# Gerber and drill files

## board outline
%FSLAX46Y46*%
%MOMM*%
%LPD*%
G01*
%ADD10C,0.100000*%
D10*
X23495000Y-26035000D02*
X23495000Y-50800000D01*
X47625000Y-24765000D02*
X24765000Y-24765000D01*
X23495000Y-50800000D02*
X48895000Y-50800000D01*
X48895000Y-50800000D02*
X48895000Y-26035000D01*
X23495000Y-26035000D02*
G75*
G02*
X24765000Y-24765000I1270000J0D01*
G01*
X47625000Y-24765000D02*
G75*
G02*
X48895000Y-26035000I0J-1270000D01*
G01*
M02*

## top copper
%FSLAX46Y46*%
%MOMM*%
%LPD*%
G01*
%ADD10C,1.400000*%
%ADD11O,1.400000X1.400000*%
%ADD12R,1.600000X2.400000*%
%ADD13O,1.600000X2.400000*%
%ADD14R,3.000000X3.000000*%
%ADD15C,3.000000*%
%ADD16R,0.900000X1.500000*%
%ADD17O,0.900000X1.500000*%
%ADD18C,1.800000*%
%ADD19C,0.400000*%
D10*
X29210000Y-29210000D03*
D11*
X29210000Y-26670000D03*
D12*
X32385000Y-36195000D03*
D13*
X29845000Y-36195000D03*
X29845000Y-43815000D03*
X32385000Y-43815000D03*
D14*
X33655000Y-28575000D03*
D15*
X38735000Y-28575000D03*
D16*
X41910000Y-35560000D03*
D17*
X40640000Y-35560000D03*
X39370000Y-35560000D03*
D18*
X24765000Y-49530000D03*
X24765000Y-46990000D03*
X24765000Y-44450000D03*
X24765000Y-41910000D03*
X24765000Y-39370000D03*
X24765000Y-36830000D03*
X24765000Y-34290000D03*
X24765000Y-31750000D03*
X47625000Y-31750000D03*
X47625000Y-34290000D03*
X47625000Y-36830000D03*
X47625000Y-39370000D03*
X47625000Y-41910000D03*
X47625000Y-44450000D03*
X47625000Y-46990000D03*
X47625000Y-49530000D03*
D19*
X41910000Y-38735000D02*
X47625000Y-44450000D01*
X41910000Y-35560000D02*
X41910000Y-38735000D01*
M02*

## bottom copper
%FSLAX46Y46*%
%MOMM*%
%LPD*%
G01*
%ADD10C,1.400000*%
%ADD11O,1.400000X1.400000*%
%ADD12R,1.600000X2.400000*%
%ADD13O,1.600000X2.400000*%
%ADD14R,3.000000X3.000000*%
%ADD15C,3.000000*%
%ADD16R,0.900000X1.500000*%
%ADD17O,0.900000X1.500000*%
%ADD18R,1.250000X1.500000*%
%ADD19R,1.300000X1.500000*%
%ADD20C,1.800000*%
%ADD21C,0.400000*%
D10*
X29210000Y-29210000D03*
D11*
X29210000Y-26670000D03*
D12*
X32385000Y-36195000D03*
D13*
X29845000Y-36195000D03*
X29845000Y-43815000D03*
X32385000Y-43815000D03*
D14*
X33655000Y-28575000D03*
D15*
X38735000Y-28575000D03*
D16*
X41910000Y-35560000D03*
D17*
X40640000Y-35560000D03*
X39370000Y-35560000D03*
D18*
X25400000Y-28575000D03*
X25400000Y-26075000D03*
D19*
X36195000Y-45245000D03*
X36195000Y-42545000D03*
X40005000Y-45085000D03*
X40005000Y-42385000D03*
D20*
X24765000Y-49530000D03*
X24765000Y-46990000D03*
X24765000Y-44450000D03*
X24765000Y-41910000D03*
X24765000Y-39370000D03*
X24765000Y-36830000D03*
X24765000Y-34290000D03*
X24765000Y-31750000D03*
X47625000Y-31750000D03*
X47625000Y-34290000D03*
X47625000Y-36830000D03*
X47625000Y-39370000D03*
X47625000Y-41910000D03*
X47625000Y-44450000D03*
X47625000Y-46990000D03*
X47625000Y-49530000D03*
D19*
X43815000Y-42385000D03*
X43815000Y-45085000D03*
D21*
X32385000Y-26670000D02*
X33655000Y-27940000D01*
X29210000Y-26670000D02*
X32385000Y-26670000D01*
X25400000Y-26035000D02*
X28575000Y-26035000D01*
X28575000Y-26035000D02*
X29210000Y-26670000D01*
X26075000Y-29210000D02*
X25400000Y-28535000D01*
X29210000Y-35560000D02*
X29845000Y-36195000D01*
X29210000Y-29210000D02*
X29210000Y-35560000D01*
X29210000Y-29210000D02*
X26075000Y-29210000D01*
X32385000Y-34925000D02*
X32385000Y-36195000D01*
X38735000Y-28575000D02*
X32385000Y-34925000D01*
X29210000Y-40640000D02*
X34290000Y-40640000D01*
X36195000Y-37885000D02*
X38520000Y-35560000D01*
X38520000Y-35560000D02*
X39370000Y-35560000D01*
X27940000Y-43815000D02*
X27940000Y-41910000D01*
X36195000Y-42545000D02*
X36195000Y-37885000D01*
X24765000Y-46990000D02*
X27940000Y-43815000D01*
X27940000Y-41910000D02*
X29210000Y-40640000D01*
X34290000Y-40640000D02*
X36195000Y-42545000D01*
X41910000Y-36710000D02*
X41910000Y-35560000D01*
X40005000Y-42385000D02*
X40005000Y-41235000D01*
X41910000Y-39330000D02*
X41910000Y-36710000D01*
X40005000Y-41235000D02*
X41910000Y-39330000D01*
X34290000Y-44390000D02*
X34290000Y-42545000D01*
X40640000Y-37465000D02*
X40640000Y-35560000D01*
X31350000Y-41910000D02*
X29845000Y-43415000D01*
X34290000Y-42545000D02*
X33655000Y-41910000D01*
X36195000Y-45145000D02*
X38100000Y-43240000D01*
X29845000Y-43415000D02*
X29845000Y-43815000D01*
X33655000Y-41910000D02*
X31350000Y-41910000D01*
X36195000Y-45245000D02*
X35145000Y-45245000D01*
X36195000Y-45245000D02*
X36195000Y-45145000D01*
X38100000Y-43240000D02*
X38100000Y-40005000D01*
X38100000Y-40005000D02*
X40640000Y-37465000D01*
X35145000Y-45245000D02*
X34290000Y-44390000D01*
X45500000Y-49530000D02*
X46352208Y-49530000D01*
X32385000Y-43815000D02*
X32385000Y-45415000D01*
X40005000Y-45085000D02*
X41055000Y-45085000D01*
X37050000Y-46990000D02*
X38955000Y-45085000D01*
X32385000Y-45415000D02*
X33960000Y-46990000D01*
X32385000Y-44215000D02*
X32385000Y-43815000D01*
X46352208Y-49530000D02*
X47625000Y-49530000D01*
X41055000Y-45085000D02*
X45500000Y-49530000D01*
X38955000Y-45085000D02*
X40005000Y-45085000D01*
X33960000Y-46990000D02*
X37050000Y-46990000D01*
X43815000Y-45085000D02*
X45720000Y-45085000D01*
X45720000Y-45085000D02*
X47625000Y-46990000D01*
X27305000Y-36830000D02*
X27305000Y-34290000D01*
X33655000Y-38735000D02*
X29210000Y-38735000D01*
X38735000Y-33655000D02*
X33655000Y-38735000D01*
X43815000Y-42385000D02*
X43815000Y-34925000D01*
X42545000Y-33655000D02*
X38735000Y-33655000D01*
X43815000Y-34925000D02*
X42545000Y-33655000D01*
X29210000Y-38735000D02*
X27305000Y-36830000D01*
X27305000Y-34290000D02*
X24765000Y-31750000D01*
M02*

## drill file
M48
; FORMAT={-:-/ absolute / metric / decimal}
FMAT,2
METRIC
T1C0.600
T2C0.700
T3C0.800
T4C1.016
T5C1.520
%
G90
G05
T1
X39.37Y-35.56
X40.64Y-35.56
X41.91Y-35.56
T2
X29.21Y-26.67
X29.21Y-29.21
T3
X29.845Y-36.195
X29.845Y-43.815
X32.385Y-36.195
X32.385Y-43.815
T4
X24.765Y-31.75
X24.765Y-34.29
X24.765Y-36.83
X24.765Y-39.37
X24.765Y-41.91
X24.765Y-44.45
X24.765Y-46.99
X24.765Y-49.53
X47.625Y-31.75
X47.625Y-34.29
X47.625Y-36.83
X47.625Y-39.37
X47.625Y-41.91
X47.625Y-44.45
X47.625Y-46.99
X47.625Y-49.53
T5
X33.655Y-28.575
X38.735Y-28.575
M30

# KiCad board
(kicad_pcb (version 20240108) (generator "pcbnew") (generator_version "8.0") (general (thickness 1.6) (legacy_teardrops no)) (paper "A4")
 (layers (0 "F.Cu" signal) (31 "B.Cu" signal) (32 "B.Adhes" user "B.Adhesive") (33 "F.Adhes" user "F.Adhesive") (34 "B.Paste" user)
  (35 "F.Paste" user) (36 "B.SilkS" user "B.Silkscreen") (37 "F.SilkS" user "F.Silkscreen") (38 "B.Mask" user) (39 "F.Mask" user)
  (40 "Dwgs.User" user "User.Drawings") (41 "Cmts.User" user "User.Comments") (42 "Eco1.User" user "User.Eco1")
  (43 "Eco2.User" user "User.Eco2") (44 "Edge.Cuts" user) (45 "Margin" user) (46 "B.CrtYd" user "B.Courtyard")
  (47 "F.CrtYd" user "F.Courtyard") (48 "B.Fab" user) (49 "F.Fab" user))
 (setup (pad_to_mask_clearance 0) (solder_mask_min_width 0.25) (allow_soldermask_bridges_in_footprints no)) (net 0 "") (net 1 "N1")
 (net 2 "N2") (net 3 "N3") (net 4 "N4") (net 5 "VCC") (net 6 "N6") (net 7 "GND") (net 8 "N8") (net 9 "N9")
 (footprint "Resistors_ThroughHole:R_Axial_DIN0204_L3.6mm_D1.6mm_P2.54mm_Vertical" (layer "F.Cu") (at 29.21 29.21 90)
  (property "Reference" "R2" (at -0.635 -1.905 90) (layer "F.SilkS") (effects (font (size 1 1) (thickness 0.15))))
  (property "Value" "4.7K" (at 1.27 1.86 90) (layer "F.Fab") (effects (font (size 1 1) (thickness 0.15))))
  (pad "1" thru_hole circle (at 0 0 90) (size 1.4 1.4) (drill 0.7) (layers "*.Cu" "*.Mask") (remove_unused_layers no) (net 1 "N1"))
  (pad "2" thru_hole oval (at 2.54 0 90) (size 1.4 1.4) (drill 0.7) (layers "*.Cu" "*.Mask") (remove_unused_layers no) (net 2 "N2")))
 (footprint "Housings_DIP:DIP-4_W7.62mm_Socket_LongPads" (layer "F.Cu") (at 32.385 36.195 -90)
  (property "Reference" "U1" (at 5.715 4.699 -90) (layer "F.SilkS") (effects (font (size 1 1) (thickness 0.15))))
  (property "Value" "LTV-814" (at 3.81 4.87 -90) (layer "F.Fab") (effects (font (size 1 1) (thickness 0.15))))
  (pad "1" thru_hole rect (at 0 0 270) (size 2.4 1.6) (drill 0.8) (layers "*.Cu" "*.Mask") (remove_unused_layers no) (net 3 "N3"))
  (pad "2" thru_hole oval (at 0 2.54 270) (size 2.4 1.6) (drill 0.8) (layers "*.Cu" "*.Mask") (remove_unused_layers no) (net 1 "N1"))
  (pad "3" thru_hole oval (at 7.62 2.54 270) (size 2.4 1.6) (drill 0.8) (layers "*.Cu" "*.Mask") (remove_unused_layers no) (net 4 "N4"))
  (pad "4" thru_hole oval (at 7.62 0 270) (size 2.4 1.6) (drill 0.8) (layers "*.Cu" "*.Mask") (remove_unused_layers no) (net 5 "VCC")))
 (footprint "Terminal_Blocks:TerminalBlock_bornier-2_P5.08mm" (layer "F.Cu") (at 33.655 28.575)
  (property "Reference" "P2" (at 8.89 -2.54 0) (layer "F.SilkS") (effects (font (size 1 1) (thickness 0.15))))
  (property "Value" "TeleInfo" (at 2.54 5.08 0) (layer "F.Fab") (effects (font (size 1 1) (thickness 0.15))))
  (pad "1" thru_hole rect (at 0 0) (size 3 3) (drill 1.52) (layers "*.Cu" "*.Mask") (remove_unused_layers no) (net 2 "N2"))
  (pad "2" thru_hole circle (at 5.08 0) (size 3 3) (drill 1.52) (layers "*.Cu" "*.Mask") (remove_unused_layers no) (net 3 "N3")))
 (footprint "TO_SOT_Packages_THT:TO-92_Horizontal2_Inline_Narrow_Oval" (layer "F.Cu") (at 41.91 35.56 180)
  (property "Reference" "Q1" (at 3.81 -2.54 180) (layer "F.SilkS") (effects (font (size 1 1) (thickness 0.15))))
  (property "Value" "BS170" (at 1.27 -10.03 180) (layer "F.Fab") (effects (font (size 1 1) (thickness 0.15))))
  (pad "1" thru_hole rect (at 0 0) (size 0.9 1.5) (drill 0.6) (layers "*.Cu" "*.Mask") (remove_unused_layers no) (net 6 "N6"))
  (pad "2" thru_hole oval (at 1.27 0) (size 0.9 1.5) (drill 0.6) (layers "*.Cu" "*.Mask") (remove_unused_layers no) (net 4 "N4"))
  (pad "3" thru_hole oval (at 2.54 0) (size 0.9 1.5) (drill 0.6) (layers "*.Cu" "*.Mask") (remove_unused_layers no) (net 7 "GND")))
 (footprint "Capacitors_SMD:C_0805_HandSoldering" (layer "B.Cu") (at 25.4 27.325 90)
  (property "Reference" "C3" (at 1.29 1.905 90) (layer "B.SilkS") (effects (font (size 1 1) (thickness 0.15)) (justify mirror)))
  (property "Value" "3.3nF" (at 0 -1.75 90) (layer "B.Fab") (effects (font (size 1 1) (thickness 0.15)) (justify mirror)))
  (pad "1" smd rect (at -1.25 0 90) (size 1.5 1.25) (layers "B.Cu" "B.Paste" "B.Mask") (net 1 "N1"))
  (pad "2" smd rect (at 1.25 0 90) (size 1.5 1.25) (layers "B.Cu" "B.Paste" "B.Mask") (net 2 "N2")))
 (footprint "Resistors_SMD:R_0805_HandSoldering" (layer "B.Cu") (at 36.195 43.895 90)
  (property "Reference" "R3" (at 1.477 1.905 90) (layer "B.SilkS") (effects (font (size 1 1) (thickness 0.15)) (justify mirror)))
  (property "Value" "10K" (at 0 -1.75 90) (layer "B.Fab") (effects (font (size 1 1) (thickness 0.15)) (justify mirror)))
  (pad "1" smd rect (at -1.35 0 90) (size 1.5 1.3) (layers "B.Cu" "B.Paste" "B.Mask") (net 4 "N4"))
  (pad "2" smd rect (at 1.35 0 90) (size 1.5 1.3) (layers "B.Cu" "B.Paste" "B.Mask") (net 7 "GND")))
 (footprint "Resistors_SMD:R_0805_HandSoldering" (layer "B.Cu") (at 40.005 43.735 90)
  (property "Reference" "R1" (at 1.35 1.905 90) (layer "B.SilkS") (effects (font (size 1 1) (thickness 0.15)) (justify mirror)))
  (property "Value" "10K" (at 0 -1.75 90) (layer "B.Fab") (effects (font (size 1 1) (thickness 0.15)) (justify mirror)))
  (pad "1" smd rect (at -1.35 0 90) (size 1.5 1.3) (layers "B.Cu" "B.Paste" "B.Mask") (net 5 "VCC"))
  (pad "2" smd rect (at 1.35 0 90) (size 1.5 1.3) (layers "B.Cu" "B.Paste" "B.Mask") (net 6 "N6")))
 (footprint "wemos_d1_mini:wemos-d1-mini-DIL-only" (layer "B.Cu") (at 36.195 40.64 90)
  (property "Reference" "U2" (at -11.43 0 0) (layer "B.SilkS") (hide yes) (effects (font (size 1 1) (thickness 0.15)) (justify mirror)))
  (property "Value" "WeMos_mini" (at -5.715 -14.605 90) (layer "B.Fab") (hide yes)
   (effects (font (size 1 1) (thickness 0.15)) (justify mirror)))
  (pad "1" thru_hole circle (at -8.89 -11.43 90) (size 1.8 1.8) (drill 1.016) (layers "*.Cu" "*.Mask") (remove_unused_layers no))
  (pad "2" thru_hole circle (at -6.35 -11.43 90) (size 1.8 1.8) (drill 1.016) (layers "*.Cu" "*.Mask") (remove_unused_layers no)
   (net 7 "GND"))
  (pad "3" thru_hole circle (at -3.81 -11.43 90) (size 1.8 1.8) (drill 1.016) (layers "*.Cu" "*.Mask") (remove_unused_layers no))
  (pad "4" thru_hole circle (at -1.27 -11.43 90) (size 1.8 1.8) (drill 1.016) (layers "*.Cu" "*.Mask") (remove_unused_layers no))
  (pad "5" thru_hole circle (at 1.27 -11.43 90) (size 1.8 1.8) (drill 1.016) (layers "*.Cu" "*.Mask") (remove_unused_layers no))
  (pad "6" thru_hole circle (at 3.81 -11.43 90) (size 1.8 1.8) (drill 1.016) (layers "*.Cu" "*.Mask") (remove_unused_layers no))
  (pad "7" thru_hole circle (at 6.35 -11.43 90) (size 1.8 1.8) (drill 1.016) (layers "*.Cu" "*.Mask") (remove_unused_layers no))
  (pad "8" thru_hole circle (at 8.89 -11.43 90) (size 1.8 1.8) (drill 1.016) (layers "*.Cu" "*.Mask") (remove_unused_layers no) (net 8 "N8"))
  (pad "9" thru_hole circle (at 8.89 11.43 90) (size 1.8 1.8) (drill 1.016) (layers "*.Cu" "*.Mask") (remove_unused_layers no))
  (pad "10" thru_hole circle (at 6.35 11.43 90) (size 1.8 1.8) (drill 1.016) (layers "*.Cu" "*.Mask") (remove_unused_layers no))
  (pad "11" thru_hole circle (at 3.81 11.43 90) (size 1.8 1.8) (drill 1.016) (layers "*.Cu" "*.Mask") (remove_unused_layers no))
  (pad "12" thru_hole circle (at 1.27 11.43 90) (size 1.8 1.8) (drill 1.016) (layers "*.Cu" "*.Mask") (remove_unused_layers no))
  (pad "13" thru_hole circle (at -1.27 11.43 90) (size 1.8 1.8) (drill 1.016) (layers "*.Cu" "*.Mask") (remove_unused_layers no))
  (pad "14" thru_hole circle (at -3.81 11.43 90) (size 1.8 1.8) (drill 1.016) (layers "*.Cu" "*.Mask") (remove_unused_layers no)
   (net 6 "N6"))
  (pad "15" thru_hole circle (at -6.35 11.43 90) (size 1.8 1.8) (drill 1.016) (layers "*.Cu" "*.Mask") (remove_unused_layers no)
   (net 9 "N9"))
  (pad "16" thru_hole circle (at -8.89 11.43 90) (size 1.8 1.8) (drill 1.016) (layers "*.Cu" "*.Mask") (remove_unused_layers no)
   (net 5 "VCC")))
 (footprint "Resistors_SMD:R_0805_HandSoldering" (layer "B.Cu") (at 43.815 43.735 -90)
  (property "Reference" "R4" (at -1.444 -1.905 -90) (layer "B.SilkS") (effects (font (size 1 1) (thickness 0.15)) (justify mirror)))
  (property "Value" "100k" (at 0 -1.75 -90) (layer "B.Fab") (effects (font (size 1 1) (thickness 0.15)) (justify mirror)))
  (pad "1" smd rect (at -1.35 0 270) (size 1.5 1.3) (layers "B.Cu" "B.Paste" "B.Mask") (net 8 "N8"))
  (pad "2" smd rect (at 1.35 0 270) (size 1.5 1.3) (layers "B.Cu" "B.Paste" "B.Mask") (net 9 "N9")))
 (gr_line (start 23.495 26.035) (end 23.495 50.8) (stroke (width 0.1) (type solid)) (layer "Edge.Cuts"))
 (gr_line (start 47.625 24.765) (end 24.765 24.765) (stroke (width 0.1) (type solid)) (layer "Edge.Cuts"))
 (gr_line (start 23.495 50.8) (end 48.895 50.8) (stroke (width 0.1) (type solid)) (layer "Edge.Cuts"))
 (gr_line (start 48.895 50.8) (end 48.895 26.035) (stroke (width 0.1) (type solid)) (layer "Edge.Cuts"))
 (gr_arc (start 23.495 26.035) (mid 23.866974 25.136974) (end 24.765 24.765) (stroke (width 0.1) (type solid)) (layer "Edge.Cuts"))
 (gr_arc (start 47.625 24.765) (mid 48.523026 25.136974) (end 48.895 26.035) (stroke (width 0.1) (type solid)) (layer "Edge.Cuts"))
 (segment (start 32.385 26.67) (end 33.655 27.94) (width 0.4) (layer "B.Cu") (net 2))
 (segment (start 29.21 26.67) (end 32.385 26.67) (width 0.4) (layer "B.Cu") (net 2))
 (segment (start 25.4 26.035) (end 28.575 26.035) (width 0.4) (layer "B.Cu") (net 2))
 (segment (start 28.575 26.035) (end 29.21 26.67) (width 0.4) (layer "B.Cu") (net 2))
 (segment (start 26.075 29.21) (end 25.4 28.535) (width 0.4) (layer "B.Cu") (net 1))
 (segment (start 29.21 35.56) (end 29.845 36.195) (width 0.4) (layer "B.Cu") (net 1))
 (segment (start 29.21 29.21) (end 29.21 35.56) (width 0.4) (layer "B.Cu") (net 1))
 (segment (start 29.21 29.21) (end 26.075 29.21) (width 0.4) (layer "B.Cu") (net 1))
 (segment (start 32.385 34.925) (end 32.385 36.195) (width 0.4) (layer "B.Cu") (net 3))
 (segment (start 38.735 28.575) (end 32.385 34.925) (width 0.4) (layer "B.Cu") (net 3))
 (segment (start 29.21 40.64) (end 34.29 40.64) (width 0.4) (layer "B.Cu") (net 7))
 (segment (start 36.195 37.885) (end 38.52 35.56) (width 0.4) (layer "B.Cu") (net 7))
 (segment (start 38.52 35.56) (end 39.37 35.56) (width 0.4) (layer "B.Cu") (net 7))
 (segment (start 27.94 43.815) (end 27.94 41.91) (width 0.4) (layer "B.Cu") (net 7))
 (segment (start 36.195 42.545) (end 36.195 37.885) (width 0.4) (layer "B.Cu") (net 7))
 (segment (start 24.765 46.99) (end 27.94 43.815) (width 0.4) (layer "B.Cu") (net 7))
 (segment (start 27.94 41.91) (end 29.21 40.64) (width 0.4) (layer "B.Cu") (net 7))
 (segment (start 34.29 40.64) (end 36.195 42.545) (width 0.4) (layer "B.Cu") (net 7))
 (segment (start 41.91 38.735) (end 47.625 44.45) (width 0.4) (layer "F.Cu") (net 6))
 (segment (start 41.91 35.56) (end 41.91 38.735) (width 0.4) (layer "F.Cu") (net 6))
 (segment (start 41.91 36.71) (end 41.91 35.56) (width 0.4) (layer "B.Cu") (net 6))
 (segment (start 40.005 42.385) (end 40.005 41.235) (width 0.4) (layer "B.Cu") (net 6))
 (segment (start 41.91 39.33) (end 41.91 36.71) (width 0.4) (layer "B.Cu") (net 6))
 (segment (start 40.005 41.235) (end 41.91 39.33) (width 0.4) (layer "B.Cu") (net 6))
 (segment (start 34.29 44.39) (end 34.29 42.545) (width 0.4) (layer "B.Cu") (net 4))
 (segment (start 40.64 37.465) (end 40.64 35.56) (width 0.4) (layer "B.Cu") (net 4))
 (segment (start 31.35 41.91) (end 29.845 43.415) (width 0.4) (layer "B.Cu") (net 4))
 (segment (start 34.29 42.545) (end 33.655 41.91) (width 0.4) (layer "B.Cu") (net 4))
 (segment (start 36.195 45.145) (end 38.1 43.24) (width 0.4) (layer "B.Cu") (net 4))
 (segment (start 29.845 43.415) (end 29.845 43.815) (width 0.4) (layer "B.Cu") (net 4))
 (segment (start 33.655 41.91) (end 31.35 41.91) (width 0.4) (layer "B.Cu") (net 4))
 (segment (start 36.195 45.245) (end 35.145 45.245) (width 0.4) (layer "B.Cu") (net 4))
 (segment (start 36.195 45.245) (end 36.195 45.145) (width 0.4) (layer "B.Cu") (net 4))
 (segment (start 38.1 43.24) (end 38.1 40.005) (width 0.4) (layer "B.Cu") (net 4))
 (segment (start 38.1 40.005) (end 40.64 37.465) (width 0.4) (layer "B.Cu") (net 4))
 (segment (start 35.145 45.245) (end 34.29 44.39) (width 0.4) (layer "B.Cu") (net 4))
 (segment (start 45.5 49.53) (end 46.352208 49.53) (width 0.4) (layer "B.Cu") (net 5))
 (segment (start 32.385 43.815) (end 32.385 45.415) (width 0.4) (layer "B.Cu") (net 5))
 (segment (start 40.005 45.085) (end 41.055 45.085) (width 0.4) (layer "B.Cu") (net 5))
 (segment (start 37.05 46.99) (end 38.955 45.085) (width 0.4) (layer "B.Cu") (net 5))
 (segment (start 32.385 45.415) (end 33.96 46.99) (width 0.4) (layer "B.Cu") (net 5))
 (segment (start 32.385 44.215) (end 32.385 43.815) (width 0.4) (layer "B.Cu") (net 5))
 (segment (start 46.352208 49.53) (end 47.625 49.53) (width 0.4) (layer "B.Cu") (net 5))
 (segment (start 41.055 45.085) (end 45.5 49.53) (width 0.4) (layer "B.Cu") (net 5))
 (segment (start 38.955 45.085) (end 40.005 45.085) (width 0.4) (layer "B.Cu") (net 5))
 (segment (start 33.96 46.99) (end 37.05 46.99) (width 0.4) (layer "B.Cu") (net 5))
 (segment (start 43.815 45.085) (end 45.72 45.085) (width 0.4) (layer "B.Cu") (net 9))
 (segment (start 45.72 45.085) (end 47.625 46.99) (width 0.4) (layer "B.Cu") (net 9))
 (segment (start 27.305 36.83) (end 27.305 34.29) (width 0.4) (layer "B.Cu") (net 8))
 (segment (start 33.655 38.735) (end 29.21 38.735) (width 0.4) (layer "B.Cu") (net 8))
 (segment (start 38.735 33.655) (end 33.655 38.735) (width 0.4) (layer "B.Cu") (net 8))
 (segment (start 43.815 42.385) (end 43.815 34.925) (width 0.4) (layer "B.Cu") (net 8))
 (segment (start 42.545 33.655) (end 38.735 33.655) (width 0.4) (layer "B.Cu") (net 8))
 (segment (start 43.815 34.925) (end 42.545 33.655) (width 0.4) (layer "B.Cu") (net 8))
 (segment (start 29.21 38.735) (end 27.305 36.83) (width 0.4) (layer "B.Cu") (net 8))
 (segment (start 27.305 34.29) (end 24.765 31.75) (width 0.4) (layer "B.Cu") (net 8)))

